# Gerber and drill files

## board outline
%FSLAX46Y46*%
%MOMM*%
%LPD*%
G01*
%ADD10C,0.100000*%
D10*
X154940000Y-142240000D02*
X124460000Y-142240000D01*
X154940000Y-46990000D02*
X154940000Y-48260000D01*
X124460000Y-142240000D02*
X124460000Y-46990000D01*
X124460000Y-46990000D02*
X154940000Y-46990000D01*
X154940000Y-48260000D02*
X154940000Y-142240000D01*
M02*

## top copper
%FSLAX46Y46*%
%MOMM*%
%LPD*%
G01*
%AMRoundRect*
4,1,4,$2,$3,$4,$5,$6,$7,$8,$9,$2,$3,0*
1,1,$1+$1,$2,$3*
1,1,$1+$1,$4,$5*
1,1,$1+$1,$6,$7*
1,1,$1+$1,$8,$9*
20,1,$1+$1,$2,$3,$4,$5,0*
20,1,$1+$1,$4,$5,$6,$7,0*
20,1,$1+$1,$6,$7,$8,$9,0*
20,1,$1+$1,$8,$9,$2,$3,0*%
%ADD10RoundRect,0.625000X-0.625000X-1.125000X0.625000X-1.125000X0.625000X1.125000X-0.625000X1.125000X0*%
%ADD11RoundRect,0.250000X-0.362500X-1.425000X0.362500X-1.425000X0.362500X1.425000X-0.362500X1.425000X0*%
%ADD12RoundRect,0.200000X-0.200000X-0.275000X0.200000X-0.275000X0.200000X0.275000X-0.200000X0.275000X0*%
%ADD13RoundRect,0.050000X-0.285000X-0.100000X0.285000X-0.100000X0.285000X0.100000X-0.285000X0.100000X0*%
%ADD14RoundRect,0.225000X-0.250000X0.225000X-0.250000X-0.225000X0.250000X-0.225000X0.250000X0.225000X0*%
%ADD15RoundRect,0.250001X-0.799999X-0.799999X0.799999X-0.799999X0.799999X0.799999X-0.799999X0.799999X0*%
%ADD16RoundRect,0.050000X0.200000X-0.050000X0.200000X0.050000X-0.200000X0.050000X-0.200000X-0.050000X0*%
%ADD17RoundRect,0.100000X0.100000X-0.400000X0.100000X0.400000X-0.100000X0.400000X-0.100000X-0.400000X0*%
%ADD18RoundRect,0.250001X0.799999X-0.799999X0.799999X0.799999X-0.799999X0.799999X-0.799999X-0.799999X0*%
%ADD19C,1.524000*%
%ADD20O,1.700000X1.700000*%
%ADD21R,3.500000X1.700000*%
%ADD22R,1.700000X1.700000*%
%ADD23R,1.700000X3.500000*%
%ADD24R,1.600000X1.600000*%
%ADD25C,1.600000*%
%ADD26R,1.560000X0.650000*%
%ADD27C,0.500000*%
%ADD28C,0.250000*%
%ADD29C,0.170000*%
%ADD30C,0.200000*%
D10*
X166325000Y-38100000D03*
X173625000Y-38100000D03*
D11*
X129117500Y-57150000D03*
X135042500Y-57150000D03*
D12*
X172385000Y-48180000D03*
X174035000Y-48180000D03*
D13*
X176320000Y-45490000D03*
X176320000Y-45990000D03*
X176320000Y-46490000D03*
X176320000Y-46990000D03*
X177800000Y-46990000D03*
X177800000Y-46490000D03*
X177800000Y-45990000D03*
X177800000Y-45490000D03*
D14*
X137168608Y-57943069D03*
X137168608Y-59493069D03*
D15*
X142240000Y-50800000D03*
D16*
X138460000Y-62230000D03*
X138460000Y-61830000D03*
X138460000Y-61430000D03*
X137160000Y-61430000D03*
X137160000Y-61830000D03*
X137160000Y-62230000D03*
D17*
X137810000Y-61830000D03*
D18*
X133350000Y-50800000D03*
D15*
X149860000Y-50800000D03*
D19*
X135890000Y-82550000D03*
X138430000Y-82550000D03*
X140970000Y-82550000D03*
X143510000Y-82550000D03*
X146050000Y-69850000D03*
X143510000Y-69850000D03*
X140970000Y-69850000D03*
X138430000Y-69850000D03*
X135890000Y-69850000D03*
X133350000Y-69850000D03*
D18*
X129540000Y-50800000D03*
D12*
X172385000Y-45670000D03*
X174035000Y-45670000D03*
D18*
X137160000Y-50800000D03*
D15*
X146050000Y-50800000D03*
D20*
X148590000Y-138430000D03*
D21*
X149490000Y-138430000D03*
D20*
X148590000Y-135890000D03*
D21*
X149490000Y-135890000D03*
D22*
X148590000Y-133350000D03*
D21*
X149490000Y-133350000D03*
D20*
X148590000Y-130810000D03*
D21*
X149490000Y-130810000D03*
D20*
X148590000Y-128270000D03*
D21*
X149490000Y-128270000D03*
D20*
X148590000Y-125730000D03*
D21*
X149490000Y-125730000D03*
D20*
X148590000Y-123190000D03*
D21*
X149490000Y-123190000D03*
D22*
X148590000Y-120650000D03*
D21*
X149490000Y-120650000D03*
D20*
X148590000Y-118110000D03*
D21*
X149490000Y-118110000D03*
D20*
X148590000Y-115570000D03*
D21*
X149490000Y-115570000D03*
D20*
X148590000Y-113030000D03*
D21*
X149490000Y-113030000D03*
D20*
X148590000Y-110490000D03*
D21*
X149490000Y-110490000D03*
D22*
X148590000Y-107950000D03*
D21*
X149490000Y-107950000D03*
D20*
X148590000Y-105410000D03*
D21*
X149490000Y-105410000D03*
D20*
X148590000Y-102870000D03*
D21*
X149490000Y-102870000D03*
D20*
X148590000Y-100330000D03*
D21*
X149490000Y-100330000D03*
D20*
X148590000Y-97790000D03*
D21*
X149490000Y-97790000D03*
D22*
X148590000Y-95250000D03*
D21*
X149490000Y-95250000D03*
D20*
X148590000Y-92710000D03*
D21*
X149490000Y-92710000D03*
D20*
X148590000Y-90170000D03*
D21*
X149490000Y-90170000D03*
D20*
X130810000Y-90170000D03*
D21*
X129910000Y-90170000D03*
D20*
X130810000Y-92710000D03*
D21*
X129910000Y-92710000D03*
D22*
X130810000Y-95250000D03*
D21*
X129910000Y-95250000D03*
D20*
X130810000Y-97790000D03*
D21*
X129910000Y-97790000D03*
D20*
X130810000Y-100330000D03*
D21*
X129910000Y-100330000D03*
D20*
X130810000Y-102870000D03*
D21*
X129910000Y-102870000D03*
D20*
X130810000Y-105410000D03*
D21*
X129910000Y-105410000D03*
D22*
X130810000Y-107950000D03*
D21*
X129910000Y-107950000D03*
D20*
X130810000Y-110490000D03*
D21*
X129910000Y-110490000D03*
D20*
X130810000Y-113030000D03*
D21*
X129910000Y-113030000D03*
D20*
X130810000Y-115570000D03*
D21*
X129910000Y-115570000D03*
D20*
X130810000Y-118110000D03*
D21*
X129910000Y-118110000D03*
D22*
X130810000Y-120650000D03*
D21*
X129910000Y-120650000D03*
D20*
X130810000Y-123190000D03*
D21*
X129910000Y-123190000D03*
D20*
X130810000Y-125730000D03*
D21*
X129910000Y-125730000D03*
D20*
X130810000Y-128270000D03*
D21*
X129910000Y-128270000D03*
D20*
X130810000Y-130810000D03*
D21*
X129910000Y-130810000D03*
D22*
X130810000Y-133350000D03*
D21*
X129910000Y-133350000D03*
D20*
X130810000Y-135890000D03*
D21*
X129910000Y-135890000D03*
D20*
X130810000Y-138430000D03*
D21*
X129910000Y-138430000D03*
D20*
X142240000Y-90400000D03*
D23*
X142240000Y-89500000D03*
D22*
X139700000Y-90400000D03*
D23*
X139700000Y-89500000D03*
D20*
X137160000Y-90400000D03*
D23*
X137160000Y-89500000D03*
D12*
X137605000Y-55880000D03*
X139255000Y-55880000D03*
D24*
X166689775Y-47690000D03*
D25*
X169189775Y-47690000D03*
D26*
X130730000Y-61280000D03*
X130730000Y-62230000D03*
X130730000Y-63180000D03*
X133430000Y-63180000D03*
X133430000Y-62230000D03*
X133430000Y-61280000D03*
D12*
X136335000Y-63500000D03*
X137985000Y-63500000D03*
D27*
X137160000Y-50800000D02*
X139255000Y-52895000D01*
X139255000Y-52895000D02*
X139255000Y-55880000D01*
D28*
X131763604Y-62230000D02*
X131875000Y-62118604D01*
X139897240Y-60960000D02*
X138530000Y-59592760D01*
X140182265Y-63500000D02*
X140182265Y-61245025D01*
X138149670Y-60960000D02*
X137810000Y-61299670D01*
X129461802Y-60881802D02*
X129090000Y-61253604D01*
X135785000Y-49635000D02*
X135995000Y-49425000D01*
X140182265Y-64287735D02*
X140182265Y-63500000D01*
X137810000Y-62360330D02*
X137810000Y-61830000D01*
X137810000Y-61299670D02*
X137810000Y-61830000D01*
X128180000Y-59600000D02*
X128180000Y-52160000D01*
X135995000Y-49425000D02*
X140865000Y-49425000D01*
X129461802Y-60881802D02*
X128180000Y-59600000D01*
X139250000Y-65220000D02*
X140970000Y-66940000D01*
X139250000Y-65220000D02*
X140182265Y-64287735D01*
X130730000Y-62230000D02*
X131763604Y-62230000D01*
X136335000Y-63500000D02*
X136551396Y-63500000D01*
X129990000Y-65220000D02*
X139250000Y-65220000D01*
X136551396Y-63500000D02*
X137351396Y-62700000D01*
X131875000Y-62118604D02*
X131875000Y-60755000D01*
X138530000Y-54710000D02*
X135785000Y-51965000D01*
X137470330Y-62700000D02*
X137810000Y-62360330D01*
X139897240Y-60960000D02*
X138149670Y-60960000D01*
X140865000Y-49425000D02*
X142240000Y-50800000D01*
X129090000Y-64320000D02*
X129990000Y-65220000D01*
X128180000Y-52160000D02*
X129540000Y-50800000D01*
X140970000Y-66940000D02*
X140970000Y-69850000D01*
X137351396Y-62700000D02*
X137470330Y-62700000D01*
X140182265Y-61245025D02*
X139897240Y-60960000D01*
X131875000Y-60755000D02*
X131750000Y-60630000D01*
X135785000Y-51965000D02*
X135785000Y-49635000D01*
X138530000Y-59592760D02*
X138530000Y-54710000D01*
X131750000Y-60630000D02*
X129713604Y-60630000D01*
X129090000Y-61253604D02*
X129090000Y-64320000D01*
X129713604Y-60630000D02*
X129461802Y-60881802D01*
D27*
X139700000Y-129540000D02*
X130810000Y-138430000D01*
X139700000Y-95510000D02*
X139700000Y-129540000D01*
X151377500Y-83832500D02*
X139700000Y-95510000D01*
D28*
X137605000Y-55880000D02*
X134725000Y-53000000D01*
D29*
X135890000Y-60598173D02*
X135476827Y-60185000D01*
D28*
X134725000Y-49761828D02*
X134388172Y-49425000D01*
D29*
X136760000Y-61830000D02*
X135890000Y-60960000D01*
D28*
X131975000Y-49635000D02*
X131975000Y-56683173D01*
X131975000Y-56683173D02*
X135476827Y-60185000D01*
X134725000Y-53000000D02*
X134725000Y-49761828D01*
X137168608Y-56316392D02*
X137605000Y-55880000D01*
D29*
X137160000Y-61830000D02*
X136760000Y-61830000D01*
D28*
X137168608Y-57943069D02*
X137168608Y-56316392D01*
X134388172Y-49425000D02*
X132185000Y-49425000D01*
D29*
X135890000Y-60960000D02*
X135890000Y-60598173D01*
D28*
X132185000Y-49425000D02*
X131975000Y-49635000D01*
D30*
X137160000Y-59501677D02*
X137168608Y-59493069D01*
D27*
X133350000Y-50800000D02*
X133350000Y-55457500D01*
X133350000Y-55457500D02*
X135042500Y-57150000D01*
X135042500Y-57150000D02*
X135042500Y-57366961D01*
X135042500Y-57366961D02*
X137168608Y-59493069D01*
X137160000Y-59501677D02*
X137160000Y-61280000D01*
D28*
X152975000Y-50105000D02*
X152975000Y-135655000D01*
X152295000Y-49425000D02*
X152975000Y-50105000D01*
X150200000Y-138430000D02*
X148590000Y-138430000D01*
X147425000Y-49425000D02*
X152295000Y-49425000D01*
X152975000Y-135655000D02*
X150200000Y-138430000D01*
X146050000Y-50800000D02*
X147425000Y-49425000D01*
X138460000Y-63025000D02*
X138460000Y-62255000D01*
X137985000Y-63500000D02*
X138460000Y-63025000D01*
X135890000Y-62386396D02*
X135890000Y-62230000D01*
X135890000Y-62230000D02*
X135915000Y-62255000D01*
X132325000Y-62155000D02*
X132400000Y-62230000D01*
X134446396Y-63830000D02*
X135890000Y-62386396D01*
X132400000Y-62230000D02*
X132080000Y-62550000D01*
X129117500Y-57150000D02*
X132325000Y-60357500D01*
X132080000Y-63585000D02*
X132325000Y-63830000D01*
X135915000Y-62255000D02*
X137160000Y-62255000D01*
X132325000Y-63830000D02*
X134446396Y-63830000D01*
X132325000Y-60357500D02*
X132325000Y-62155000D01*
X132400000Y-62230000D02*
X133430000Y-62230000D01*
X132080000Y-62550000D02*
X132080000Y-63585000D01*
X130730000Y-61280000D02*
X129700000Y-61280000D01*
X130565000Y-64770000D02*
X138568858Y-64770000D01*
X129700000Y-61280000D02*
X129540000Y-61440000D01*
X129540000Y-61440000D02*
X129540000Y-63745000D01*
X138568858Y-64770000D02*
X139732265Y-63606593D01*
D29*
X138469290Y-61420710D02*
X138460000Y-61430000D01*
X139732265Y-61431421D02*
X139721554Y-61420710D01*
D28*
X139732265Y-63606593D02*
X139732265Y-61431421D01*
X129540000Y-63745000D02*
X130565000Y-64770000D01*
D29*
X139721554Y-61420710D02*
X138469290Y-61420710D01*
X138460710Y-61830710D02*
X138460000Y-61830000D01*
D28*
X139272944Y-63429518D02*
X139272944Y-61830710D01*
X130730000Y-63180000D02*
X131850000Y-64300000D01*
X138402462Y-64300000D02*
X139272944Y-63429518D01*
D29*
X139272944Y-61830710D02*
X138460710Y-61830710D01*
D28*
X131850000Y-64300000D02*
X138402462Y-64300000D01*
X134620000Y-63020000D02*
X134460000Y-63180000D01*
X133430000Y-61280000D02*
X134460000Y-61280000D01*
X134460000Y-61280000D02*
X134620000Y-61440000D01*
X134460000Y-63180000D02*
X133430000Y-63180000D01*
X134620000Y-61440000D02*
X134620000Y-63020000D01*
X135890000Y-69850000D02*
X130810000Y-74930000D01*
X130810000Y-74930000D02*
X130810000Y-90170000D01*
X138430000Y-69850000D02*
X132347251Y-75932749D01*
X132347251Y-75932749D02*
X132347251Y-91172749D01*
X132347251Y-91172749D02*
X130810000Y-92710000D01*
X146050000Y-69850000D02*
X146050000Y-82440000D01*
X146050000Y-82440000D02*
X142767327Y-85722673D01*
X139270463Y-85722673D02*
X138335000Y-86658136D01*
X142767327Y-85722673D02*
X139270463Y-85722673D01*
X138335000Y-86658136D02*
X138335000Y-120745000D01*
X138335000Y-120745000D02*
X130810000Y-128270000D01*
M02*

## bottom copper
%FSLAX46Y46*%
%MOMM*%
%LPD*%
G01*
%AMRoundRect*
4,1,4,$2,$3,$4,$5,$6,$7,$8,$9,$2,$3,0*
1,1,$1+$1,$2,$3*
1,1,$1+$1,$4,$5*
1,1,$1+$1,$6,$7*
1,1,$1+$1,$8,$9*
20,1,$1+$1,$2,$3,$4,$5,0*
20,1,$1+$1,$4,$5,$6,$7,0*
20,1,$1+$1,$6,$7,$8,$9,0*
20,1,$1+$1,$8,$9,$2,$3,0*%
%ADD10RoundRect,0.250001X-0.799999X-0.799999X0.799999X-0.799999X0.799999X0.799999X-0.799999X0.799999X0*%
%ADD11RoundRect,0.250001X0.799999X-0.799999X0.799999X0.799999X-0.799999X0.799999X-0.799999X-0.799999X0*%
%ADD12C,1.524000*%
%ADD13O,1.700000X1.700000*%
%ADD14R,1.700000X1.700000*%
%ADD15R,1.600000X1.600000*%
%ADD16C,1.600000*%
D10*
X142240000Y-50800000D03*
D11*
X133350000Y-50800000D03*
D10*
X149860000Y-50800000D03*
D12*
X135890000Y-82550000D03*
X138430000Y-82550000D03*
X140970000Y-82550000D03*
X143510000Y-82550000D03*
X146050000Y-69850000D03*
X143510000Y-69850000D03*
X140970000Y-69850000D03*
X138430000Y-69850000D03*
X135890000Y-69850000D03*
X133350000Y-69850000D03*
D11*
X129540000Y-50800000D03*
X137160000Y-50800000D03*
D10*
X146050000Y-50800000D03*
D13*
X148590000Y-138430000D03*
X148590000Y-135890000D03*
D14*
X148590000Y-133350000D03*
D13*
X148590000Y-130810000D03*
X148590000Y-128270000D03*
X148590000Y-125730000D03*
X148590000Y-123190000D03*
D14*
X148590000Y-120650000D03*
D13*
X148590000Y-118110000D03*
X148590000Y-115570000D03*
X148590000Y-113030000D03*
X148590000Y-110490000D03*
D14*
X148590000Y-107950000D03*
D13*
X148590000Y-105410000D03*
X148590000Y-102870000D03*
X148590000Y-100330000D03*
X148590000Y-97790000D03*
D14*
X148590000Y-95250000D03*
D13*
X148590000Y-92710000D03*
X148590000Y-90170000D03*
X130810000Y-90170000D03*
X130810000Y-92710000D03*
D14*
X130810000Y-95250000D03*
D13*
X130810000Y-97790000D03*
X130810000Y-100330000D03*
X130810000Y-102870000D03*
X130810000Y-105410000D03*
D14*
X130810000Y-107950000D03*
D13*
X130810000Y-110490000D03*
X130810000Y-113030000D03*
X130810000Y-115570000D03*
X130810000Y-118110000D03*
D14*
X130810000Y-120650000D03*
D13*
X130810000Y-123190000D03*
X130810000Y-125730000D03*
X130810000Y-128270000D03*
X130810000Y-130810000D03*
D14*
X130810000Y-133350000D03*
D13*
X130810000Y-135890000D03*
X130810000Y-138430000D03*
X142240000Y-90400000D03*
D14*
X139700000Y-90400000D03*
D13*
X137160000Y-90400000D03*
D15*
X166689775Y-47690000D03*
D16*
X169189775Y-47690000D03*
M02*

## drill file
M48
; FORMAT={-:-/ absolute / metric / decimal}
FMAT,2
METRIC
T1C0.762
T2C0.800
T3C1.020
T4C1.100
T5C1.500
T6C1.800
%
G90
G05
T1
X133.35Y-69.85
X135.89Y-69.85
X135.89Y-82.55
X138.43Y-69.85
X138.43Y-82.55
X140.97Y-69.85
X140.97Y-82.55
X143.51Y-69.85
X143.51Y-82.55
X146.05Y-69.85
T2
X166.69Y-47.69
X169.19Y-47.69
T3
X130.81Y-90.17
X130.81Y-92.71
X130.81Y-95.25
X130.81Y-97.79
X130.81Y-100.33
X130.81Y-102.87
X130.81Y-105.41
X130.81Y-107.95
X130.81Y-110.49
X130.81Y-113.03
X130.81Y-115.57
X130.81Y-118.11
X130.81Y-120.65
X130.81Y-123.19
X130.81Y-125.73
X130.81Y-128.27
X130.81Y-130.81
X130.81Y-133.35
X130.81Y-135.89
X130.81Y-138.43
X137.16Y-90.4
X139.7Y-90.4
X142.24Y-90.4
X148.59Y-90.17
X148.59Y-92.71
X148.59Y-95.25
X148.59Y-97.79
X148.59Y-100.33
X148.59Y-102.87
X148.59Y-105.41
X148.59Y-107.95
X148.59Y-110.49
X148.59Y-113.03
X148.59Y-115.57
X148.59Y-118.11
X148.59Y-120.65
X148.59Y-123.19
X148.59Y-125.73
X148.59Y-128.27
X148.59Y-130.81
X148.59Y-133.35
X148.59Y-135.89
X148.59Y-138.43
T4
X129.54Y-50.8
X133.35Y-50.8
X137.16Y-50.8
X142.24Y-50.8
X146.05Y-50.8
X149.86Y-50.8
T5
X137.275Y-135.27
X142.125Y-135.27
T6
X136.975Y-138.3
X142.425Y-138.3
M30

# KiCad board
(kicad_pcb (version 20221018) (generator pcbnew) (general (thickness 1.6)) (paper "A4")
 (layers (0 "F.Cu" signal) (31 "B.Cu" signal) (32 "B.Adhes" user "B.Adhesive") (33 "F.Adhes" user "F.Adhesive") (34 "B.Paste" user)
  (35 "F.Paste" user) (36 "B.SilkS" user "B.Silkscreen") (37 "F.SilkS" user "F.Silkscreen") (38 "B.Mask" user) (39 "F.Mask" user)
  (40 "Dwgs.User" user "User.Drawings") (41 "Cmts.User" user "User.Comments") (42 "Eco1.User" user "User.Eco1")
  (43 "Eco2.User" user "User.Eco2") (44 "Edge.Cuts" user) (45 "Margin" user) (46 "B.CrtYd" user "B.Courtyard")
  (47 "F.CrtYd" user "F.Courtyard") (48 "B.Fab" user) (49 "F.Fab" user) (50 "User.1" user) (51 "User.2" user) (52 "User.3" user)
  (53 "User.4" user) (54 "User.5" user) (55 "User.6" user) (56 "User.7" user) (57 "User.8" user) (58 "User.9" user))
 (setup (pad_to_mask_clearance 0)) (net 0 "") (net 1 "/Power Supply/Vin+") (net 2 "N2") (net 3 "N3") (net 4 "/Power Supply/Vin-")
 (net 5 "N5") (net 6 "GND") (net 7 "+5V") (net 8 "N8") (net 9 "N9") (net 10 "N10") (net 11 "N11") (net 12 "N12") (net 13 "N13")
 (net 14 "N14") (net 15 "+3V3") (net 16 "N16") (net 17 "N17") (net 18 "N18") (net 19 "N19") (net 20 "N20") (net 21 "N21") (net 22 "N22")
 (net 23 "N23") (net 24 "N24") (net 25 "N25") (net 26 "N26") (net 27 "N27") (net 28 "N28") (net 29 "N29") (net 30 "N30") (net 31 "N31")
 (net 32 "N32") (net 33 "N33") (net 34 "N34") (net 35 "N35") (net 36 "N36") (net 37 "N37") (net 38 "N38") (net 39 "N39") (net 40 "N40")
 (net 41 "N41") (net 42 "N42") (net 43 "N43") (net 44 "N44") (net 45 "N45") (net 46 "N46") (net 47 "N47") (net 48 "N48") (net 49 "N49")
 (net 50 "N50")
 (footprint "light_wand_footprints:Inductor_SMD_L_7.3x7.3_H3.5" (layer "F.Cu") (at 169.975 38.1)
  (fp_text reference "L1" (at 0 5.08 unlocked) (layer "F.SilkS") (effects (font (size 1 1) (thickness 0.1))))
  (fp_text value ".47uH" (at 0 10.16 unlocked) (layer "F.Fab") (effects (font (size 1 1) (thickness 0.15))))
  (pad "1" smd roundrect (at -3.65 0) (size 2.5 3.5) (layers "F.Cu" "F.Paste" "F.Mask") (roundrect_rratio 0.25) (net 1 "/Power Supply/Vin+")
   (thermal_bridge_angle 45))
  (pad "2" smd roundrect (at 3.65 0) (size 2.5 3.5) (layers "F.Cu" "F.Paste" "F.Mask") (roundrect_rratio 0.25) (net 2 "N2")
   (thermal_bridge_angle 45)))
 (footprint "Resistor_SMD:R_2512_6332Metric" (layer "F.Cu") (at 132.08 57.15)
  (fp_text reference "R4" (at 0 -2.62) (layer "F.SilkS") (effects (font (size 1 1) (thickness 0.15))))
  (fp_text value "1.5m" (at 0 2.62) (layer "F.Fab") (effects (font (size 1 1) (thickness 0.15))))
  (pad "1" smd roundrect (at -2.9625 0) (size 1.225 3.35) (layers "F.Cu" "F.Paste" "F.Mask") (roundrect_rratio 0.204082) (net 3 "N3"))
  (pad "2" smd roundrect (at 2.9625 0) (size 1.225 3.35) (layers "F.Cu" "F.Paste" "F.Mask") (roundrect_rratio 0.204082)
   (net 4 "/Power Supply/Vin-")))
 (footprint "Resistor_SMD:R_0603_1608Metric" (layer "F.Cu") (at 173.21 48.18)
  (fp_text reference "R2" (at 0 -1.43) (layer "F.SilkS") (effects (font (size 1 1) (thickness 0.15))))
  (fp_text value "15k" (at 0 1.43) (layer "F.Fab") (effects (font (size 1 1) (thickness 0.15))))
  (pad "1" smd roundrect (at -0.825 0) (size 0.8 0.95) (layers "F.Cu" "F.Paste" "F.Mask") (roundrect_rratio 0.25) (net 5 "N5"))
  (pad "2" smd roundrect (at 0.825 0) (size 0.8 0.95) (layers "F.Cu" "F.Paste" "F.Mask") (roundrect_rratio 0.25) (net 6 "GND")))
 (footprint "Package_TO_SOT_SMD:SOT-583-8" (layer "F.Cu") (at 177.06 46.24)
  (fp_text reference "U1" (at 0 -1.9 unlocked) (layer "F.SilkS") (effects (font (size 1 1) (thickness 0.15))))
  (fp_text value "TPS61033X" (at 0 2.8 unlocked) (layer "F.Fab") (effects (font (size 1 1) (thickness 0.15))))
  (pad "1" smd roundrect (at -0.74 -0.75) (size 0.67 0.3) (layers "F.Cu" "F.Paste" "F.Mask") (roundrect_rratio 0.1666666667)
   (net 1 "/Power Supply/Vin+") (thermal_bridge_angle 45))
  (pad "2" smd roundrect (at -0.74 -0.25) (size 0.67 0.3) (layers "F.Cu" "F.Paste" "F.Mask") (roundrect_rratio 0.1666666667)
   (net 1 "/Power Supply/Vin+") (thermal_bridge_angle 45))
  (pad "3" smd roundrect (at -0.74 0.25) (size 0.67 0.3) (layers "F.Cu" "F.Paste" "F.Mask") (roundrect_rratio 0.1666666667)
   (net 1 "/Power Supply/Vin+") (thermal_bridge_angle 45))
  (pad "4" smd roundrect (at -0.74 0.75) (size 0.67 0.3) (layers "F.Cu" "F.Paste" "F.Mask") (roundrect_rratio 0.1666666667) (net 6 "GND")
   (thermal_bridge_angle 45))
  (pad "5" smd roundrect (at 0.74 0.75) (size 0.67 0.3) (layers "F.Cu" "F.Paste" "F.Mask") (roundrect_rratio 0.1666666667) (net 5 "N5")
   (thermal_bridge_angle 45))
  (pad "6" smd roundrect (at 0.74 0.25) (size 0.67 0.3) (layers "F.Cu" "F.Paste" "F.Mask") (roundrect_rratio 0.1666666667) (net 6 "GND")
   (thermal_bridge_angle 45))
  (pad "7" smd roundrect (at 0.74 -0.25) (size 0.67 0.3) (layers "F.Cu" "F.Paste" "F.Mask") (roundrect_rratio 0.1666666667) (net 2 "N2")
   (thermal_bridge_angle 45))
  (pad "8" smd roundrect (at 0.74 -0.75) (size 0.67 0.3) (layers "F.Cu" "F.Paste" "F.Mask") (roundrect_rratio 0.1666666667) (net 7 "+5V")
   (thermal_bridge_angle 45)))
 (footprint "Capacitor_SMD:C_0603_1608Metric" (layer "F.Cu") (at 137.168608 58.718069 -90)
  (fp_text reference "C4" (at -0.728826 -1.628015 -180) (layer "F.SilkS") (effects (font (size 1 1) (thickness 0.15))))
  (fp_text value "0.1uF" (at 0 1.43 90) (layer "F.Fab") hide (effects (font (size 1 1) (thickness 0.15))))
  (pad "1" smd roundrect (at -0.775 0 270) (size 0.9 0.95) (layers "F.Cu" "F.Paste" "F.Mask") (roundrect_rratio 0.25) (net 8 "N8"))
  (pad "2" smd roundrect (at 0.775 0 270) (size 0.9 0.95) (layers "F.Cu" "F.Paste" "F.Mask") (roundrect_rratio 0.25)
   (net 4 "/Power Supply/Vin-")))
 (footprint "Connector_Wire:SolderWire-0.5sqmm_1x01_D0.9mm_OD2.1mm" (layer "F.Cu") (at 142.24 50.8)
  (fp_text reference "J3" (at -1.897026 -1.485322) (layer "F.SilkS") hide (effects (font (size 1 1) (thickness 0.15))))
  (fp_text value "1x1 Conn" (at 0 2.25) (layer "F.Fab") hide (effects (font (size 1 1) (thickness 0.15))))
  (pad "1" thru_hole roundrect (at 0 0) (size 2.1 2.1) (drill 1.1) (layers "*.Cu" "*.Mask") (roundrect_rratio 0.119048) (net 6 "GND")))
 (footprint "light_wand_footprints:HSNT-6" (layer "F.Cu") (at 137.81 61.83 180)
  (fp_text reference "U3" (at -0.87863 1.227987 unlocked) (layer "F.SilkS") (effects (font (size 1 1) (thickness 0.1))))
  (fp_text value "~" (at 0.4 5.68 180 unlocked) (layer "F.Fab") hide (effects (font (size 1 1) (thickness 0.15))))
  (pad "1" smd roundrect (at -0.65 -0.4 90) (size 0.2 0.5) (layers "F.Cu" "F.Paste" "F.Mask") (roundrect_rratio 0.25) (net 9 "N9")
   (thermal_bridge_angle 45))
  (pad "2" smd roundrect (at -0.65 0 90) (size 0.2 0.5) (layers "F.Cu" "F.Paste" "F.Mask") (roundrect_rratio 0.25) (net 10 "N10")
   (thermal_bridge_angle 45))
  (pad "3" smd roundrect (at -0.65 0.4 90) (size 0.2 0.5) (layers "F.Cu" "F.Paste" "F.Mask") (roundrect_rratio 0.25) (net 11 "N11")
   (thermal_bridge_angle 45))
  (pad "4" smd roundrect (at 0.65 0.4 90) (size 0.2 0.5) (layers "F.Cu" "F.Paste" "F.Mask") (roundrect_rratio 0.25)
   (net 4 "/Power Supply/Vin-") (thermal_bridge_angle 45))
  (pad "5" smd roundrect (at 0.65 0 90) (size 0.2 0.5) (layers "F.Cu" "F.Paste" "F.Mask") (roundrect_rratio 0.25) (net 8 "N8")
   (thermal_bridge_angle 45))
  (pad "6" smd roundrect (at 0.65 -0.4 90) (size 0.2 0.5) (layers "F.Cu" "F.Paste" "F.Mask") (roundrect_rratio 0.25) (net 3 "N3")
   (thermal_bridge_angle 45))
  (pad "7" smd roundrect (at 0 0 90) (size 1 0.4) (layers "F.Cu" "F.Paste" "F.Mask") (roundrect_rratio 0.25) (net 6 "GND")
   (thermal_bridge_angle 45)))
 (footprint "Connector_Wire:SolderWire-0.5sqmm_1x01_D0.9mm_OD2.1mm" (layer "F.Cu") (at 133.35 50.8 90)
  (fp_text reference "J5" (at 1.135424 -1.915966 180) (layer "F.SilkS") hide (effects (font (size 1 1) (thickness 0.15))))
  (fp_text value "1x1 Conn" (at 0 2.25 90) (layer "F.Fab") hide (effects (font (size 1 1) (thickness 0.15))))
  (pad "1" thru_hole roundrect (at 0 0 90) (size 2.1 2.1) (drill 1.1) (layers "*.Cu" "*.Mask") (roundrect_rratio 0.119048)
   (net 4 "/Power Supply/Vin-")))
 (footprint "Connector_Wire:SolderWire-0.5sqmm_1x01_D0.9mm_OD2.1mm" (layer "F.Cu") (at 149.86 50.8)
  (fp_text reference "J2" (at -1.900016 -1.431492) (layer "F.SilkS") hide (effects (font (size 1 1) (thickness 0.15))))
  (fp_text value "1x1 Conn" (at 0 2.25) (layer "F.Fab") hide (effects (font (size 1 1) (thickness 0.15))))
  (pad "1" thru_hole roundrect (at 0 0) (size 2.1 2.1) (drill 1.1) (layers "*.Cu" "*.Mask") (roundrect_rratio 0.119048) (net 7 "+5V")))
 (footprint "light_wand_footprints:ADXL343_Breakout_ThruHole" (layer "F.Cu") (at 151.13 74.93 90)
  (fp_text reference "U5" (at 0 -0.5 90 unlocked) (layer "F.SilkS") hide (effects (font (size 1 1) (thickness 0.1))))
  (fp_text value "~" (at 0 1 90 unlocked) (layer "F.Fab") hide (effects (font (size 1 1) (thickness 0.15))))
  (pad "1" thru_hole circle (at -7.62 -15.24 90) (size 1.524 1.524) (drill 0.762) (layers "*.Cu" "*.Mask") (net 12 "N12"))
  (pad "2" thru_hole circle (at -7.62 -12.7 90) (size 1.524 1.524) (drill 0.762) (layers "*.Cu" "*.Mask") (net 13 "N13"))
  (pad "3" thru_hole circle (at -7.62 -10.16 90) (size 1.524 1.524) (drill 0.762) (layers "*.Cu" "*.Mask") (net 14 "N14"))
  (pad "4" thru_hole circle (at -7.62 -7.62 90) (size 1.524 1.524) (drill 0.762) (layers "*.Cu" "*.Mask") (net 6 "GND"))
  (pad "5" thru_hole circle (at 5.08 -5.08 90) (size 1.524 1.524) (drill 0.762) (layers "*.Cu" "*.Mask") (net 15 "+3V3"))
  (pad "6" thru_hole circle (at 5.08 -7.62 90) (size 1.524 1.524) (drill 0.762) (layers "*.Cu" "*.Mask") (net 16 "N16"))
  (pad "7" thru_hole circle (at 5.08 -10.16 90) (size 1.524 1.524) (drill 0.762) (layers "*.Cu" "*.Mask") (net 6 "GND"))
  (pad "8" thru_hole circle (at 5.08 -12.7 90) (size 1.524 1.524) (drill 0.762) (layers "*.Cu" "*.Mask") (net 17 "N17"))
  (pad "9" thru_hole circle (at 5.08 -15.24 90) (size 1.524 1.524) (drill 0.762) (layers "*.Cu" "*.Mask") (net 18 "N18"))
  (pad "10" thru_hole circle (at 5.08 -17.78 90) (size 1.524 1.524) (drill 0.762) (layers "*.Cu" "*.Mask") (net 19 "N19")))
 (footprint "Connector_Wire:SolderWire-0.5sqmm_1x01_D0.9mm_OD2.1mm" (layer "F.Cu") (at 129.54 50.8 90)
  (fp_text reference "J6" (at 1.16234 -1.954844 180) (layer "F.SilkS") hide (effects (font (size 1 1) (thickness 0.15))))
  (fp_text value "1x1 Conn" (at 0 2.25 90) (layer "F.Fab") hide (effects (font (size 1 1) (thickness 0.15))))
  (pad "1" thru_hole roundrect (at 0 0 90) (size 2.1 2.1) (drill 1.1) (layers "*.Cu" "*.Mask") (roundrect_rratio 0.119048) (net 6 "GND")))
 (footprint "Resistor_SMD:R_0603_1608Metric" (layer "F.Cu") (at 173.21 45.67)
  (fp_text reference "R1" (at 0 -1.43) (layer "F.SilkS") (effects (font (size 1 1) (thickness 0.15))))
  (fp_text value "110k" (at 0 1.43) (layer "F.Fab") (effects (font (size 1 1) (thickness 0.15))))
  (pad "1" smd roundrect (at -0.825 0) (size 0.8 0.95) (layers "F.Cu" "F.Paste" "F.Mask") (roundrect_rratio 0.25) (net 7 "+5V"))
  (pad "2" smd roundrect (at 0.825 0) (size 0.8 0.95) (layers "F.Cu" "F.Paste" "F.Mask") (roundrect_rratio 0.25) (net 5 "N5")))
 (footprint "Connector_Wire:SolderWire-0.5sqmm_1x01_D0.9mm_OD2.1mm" (layer "F.Cu") (at 137.16 50.8 90)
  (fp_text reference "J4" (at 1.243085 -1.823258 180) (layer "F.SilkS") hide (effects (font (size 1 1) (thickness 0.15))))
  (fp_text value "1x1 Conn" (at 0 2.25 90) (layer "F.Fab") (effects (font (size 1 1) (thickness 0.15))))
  (pad "1" thru_hole roundrect (at 0 0 90) (size 2.1 2.1) (drill 1.1) (layers "*.Cu" "*.Mask") (roundrect_rratio 0.119048)
   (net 1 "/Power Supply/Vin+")))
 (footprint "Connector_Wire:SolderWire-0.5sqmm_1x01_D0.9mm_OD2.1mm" (layer "F.Cu") (at 146.05 50.8)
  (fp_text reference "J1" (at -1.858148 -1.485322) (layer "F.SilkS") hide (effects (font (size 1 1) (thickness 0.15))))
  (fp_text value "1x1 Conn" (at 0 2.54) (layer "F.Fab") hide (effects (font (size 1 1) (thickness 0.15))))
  (pad "1" thru_hole roundrect (at 0 0) (size 2.1 2.1) (drill 1.1) (layers "*.Cu" "*.Mask") (roundrect_rratio 0.119048) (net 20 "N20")))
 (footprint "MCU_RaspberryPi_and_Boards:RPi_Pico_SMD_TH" (layer "F.Cu") (at 139.7 114.3 180)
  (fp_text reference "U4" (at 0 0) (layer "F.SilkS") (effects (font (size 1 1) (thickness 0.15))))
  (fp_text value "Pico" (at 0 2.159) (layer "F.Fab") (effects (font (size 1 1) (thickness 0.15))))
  (pad "" np_thru_hole oval (at -2.725 -24 180) (size 1.8 1.8) (drill 1.8) (layers "*.Cu" "*.Mask"))
  (pad "" np_thru_hole oval (at -2.425 -20.97 180) (size 1.5 1.5) (drill 1.5) (layers "*.Cu" "*.Mask"))
  (pad "" np_thru_hole oval (at 2.425 -20.97 180) (size 1.5 1.5) (drill 1.5) (layers "*.Cu" "*.Mask"))
  (pad "" np_thru_hole oval (at 2.725 -24 180) (size 1.8 1.8) (drill 1.8) (layers "*.Cu" "*.Mask"))
  (pad "1" thru_hole oval (at -8.89 -24.13 180) (size 1.7 1.7) (drill 1.02) (layers "*.Cu" "*.Mask") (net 20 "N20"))
  (pad "1" smd rect (at -8.89 -24.13 180) (size 3.5 1.7) (drill (offset -0.9 0)) (layers "F.Cu" "F.Mask") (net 20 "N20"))
  (pad "2" thru_hole oval (at -8.89 -21.59 180) (size 1.7 1.7) (drill 1.02) (layers "*.Cu" "*.Mask") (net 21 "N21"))
  (pad "2" smd rect (at -8.89 -21.59 180) (size 3.5 1.7) (drill (offset -0.9 0)) (layers "F.Cu" "F.Mask") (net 21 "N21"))
  (pad "3" thru_hole rect (at -8.89 -19.05 180) (size 1.7 1.7) (drill 1.02) (layers "*.Cu" "*.Mask") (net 6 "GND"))
  (pad "3" smd rect (at -8.89 -19.05 180) (size 3.5 1.7) (drill (offset -0.9 0)) (layers "F.Cu" "F.Mask") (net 6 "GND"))
  (pad "4" thru_hole oval (at -8.89 -16.51 180) (size 1.7 1.7) (drill 1.02) (layers "*.Cu" "*.Mask") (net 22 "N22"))
  (pad "4" smd rect (at -8.89 -16.51 180) (size 3.5 1.7) (drill (offset -0.9 0)) (layers "F.Cu" "F.Mask") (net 22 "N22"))
  (pad "5" thru_hole oval (at -8.89 -13.97 180) (size 1.7 1.7) (drill 1.02) (layers "*.Cu" "*.Mask") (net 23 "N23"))
  (pad "5" smd rect (at -8.89 -13.97 180) (size 3.5 1.7) (drill (offset -0.9 0)) (layers "F.Cu" "F.Mask") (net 23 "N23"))
  (pad "6" thru_hole oval (at -8.89 -11.43 180) (size 1.7 1.7) (drill 1.02) (layers "*.Cu" "*.Mask") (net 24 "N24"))
  (pad "6" smd rect (at -8.89 -11.43 180) (size 3.5 1.7) (drill (offset -0.9 0)) (layers "F.Cu" "F.Mask") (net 24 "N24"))
  (pad "7" thru_hole oval (at -8.89 -8.89 180) (size 1.7 1.7) (drill 1.02) (layers "*.Cu" "*.Mask") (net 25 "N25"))
  (pad "7" smd rect (at -8.89 -8.89 180) (size 3.5 1.7) (drill (offset -0.9 0)) (layers "F.Cu" "F.Mask") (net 25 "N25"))
  (pad "8" thru_hole rect (at -8.89 -6.35 180) (size 1.7 1.7) (drill 1.02) (layers "*.Cu" "*.Mask") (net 6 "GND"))
  (pad "8" smd rect (at -8.89 -6.35 180) (size 3.5 1.7) (drill (offset -0.9 0)) (layers "F.Cu" "F.Mask") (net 6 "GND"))
  (pad "9" thru_hole oval (at -8.89 -3.81 180) (size 1.7 1.7) (drill 1.02) (layers "*.Cu" "*.Mask") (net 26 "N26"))
  (pad "9" smd rect (at -8.89 -3.81 180) (size 3.5 1.7) (drill (offset -0.9 0)) (layers "F.Cu" "F.Mask") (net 26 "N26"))
  (pad "10" thru_hole oval (at -8.89 -1.27 180) (size 1.7 1.7) (drill 1.02) (layers "*.Cu" "*.Mask") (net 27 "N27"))
  (pad "10" smd rect (at -8.89 -1.27 180) (size 3.5 1.7) (drill (offset -0.9 0)) (layers "F.Cu" "F.Mask") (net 27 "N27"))
  (pad "11" thru_hole oval (at -8.89 1.27 180) (size 1.7 1.7) (drill 1.02) (layers "*.Cu" "*.Mask") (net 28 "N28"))
  (pad "11" smd rect (at -8.89 1.27 180) (size 3.5 1.7) (drill (offset -0.9 0)) (layers "F.Cu" "F.Mask") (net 28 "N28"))
  (pad "12" thru_hole oval (at -8.89 3.81 180) (size 1.7 1.7) (drill 1.02) (layers "*.Cu" "*.Mask") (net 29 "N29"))
  (pad "12" smd rect (at -8.89 3.81 180) (size 3.5 1.7) (drill (offset -0.9 0)) (layers "F.Cu" "F.Mask") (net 29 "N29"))
  (pad "13" thru_hole rect (at -8.89 6.35 180) (size 1.7 1.7) (drill 1.02) (layers "*.Cu" "*.Mask") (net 6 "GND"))
  (pad "13" smd rect (at -8.89 6.35 180) (size 3.5 1.7) (drill (offset -0.9 0)) (layers "F.Cu" "F.Mask") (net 6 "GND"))
  (pad "14" thru_hole oval (at -8.89 8.89 180) (size 1.7 1.7) (drill 1.02) (layers "*.Cu" "*.Mask") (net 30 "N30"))
  (pad "14" smd rect (at -8.89 8.89 180) (size 3.5 1.7) (drill (offset -0.9 0)) (layers "F.Cu" "F.Mask") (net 30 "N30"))
  (pad "15" thru_hole oval (at -8.89 11.43 180) (size 1.7 1.7) (drill 1.02) (layers "*.Cu" "*.Mask") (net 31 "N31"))
  (pad "15" smd rect (at -8.89 11.43 180) (size 3.5 1.7) (drill (offset -0.9 0)) (layers "F.Cu" "F.Mask") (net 31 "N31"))
  (pad "16" thru_hole oval (at -8.89 13.97 180) (size 1.7 1.7) (drill 1.02) (layers "*.Cu" "*.Mask") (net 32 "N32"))
  (pad "16" smd rect (at -8.89 13.97 180) (size 3.5 1.7) (drill (offset -0.9 0)) (layers "F.Cu" "F.Mask") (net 32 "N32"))
  (pad "17" thru_hole oval (at -8.89 16.51 180) (size 1.7 1.7) (drill 1.02) (layers "*.Cu" "*.Mask") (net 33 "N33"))
  (pad "17" smd rect (at -8.89 16.51 180) (size 3.5 1.7) (drill (offset -0.9 0)) (layers "F.Cu" "F.Mask") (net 33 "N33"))
  (pad "18" thru_hole rect (at -8.89 19.05 180) (size 1.7 1.7) (drill 1.02) (layers "*.Cu" "*.Mask") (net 6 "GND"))
  (pad "18" smd rect (at -8.89 19.05 180) (size 3.5 1.7) (drill (offset -0.9 0)) (layers "F.Cu" "F.Mask") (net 6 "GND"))
  (pad "19" thru_hole oval (at -8.89 21.59 180) (size 1.7 1.7) (drill 1.02) (layers "*.Cu" "*.Mask") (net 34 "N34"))
  (pad "19" smd rect (at -8.89 21.59 180) (size 3.5 1.7) (drill (offset -0.9 0)) (layers "F.Cu" "F.Mask") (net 34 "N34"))
  (pad "20" thru_hole oval (at -8.89 24.13 180) (size 1.7 1.7) (drill 1.02) (layers "*.Cu" "*.Mask") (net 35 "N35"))
  (pad "20" smd rect (at -8.89 24.13 180) (size 3.5 1.7) (drill (offset -0.9 0)) (layers "F.Cu" "F.Mask") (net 35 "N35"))
  (pad "21" thru_hole oval (at 8.89 24.13 180) (size 1.7 1.7) (drill 1.02) (layers "*.Cu" "*.Mask") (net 18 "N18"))
  (pad "21" smd rect (at 8.89 24.13 180) (size 3.5 1.7) (drill (offset 0.9 0)) (layers "F.Cu" "F.Mask") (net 18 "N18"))
  (pad "22" thru_hole oval (at 8.89 21.59 180) (size 1.7 1.7) (drill 1.02) (layers "*.Cu" "*.Mask") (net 17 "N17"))
  (pad "22" smd rect (at 8.89 21.59 180) (size 3.5 1.7) (drill (offset 0.9 0)) (layers "F.Cu" "F.Mask") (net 17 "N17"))
  (pad "23" thru_hole rect (at 8.89 19.05 180) (size 1.7 1.7) (drill 1.02) (layers "*.Cu" "*.Mask") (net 6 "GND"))
  (pad "23" smd rect (at 8.89 19.05 180) (size 3.5 1.7) (drill (offset 0.9 0)) (layers "F.Cu" "F.Mask") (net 6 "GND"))
  (pad "24" thru_hole oval (at 8.89 16.51 180) (size 1.7 1.7) (drill 1.02) (layers "*.Cu" "*.Mask") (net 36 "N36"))
  (pad "24" smd rect (at 8.89 16.51 180) (size 3.5 1.7) (drill (offset 0.9 0)) (layers "F.Cu" "F.Mask") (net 36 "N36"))
  (pad "25" thru_hole oval (at 8.89 13.97 180) (size 1.7 1.7) (drill 1.02) (layers "*.Cu" "*.Mask") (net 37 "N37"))
  (pad "25" smd rect (at 8.89 13.97 180) (size 3.5 1.7) (drill (offset 0.9 0)) (layers "F.Cu" "F.Mask") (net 37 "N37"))
  (pad "26" thru_hole oval (at 8.89 11.43 180) (size 1.7 1.7) (drill 1.02) (layers "*.Cu" "*.Mask") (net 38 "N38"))
  (pad "26" smd rect (at 8.89 11.43 180) (size 3.5 1.7) (drill (offset 0.9 0)) (layers "F.Cu" "F.Mask") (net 38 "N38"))
  (pad "27" thru_hole oval (at 8.89 8.89 180) (size 1.7 1.7) (drill 1.02) (layers "*.Cu" "*.Mask") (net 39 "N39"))
  (pad "27" smd rect (at 8.89 8.89 180) (size 3.5 1.7) (drill (offset 0.9 0)) (layers "F.Cu" "F.Mask") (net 39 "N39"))
  (pad "28" thru_hole rect (at 8.89 6.35 180) (size 1.7 1.7) (drill 1.02) (layers "*.Cu" "*.Mask") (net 6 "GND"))
  (pad "28" smd rect (at 8.89 6.35 180) (size 3.5 1.7) (drill (offset 0.9 0)) (layers "F.Cu" "F.Mask") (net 6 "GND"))
  (pad "29" thru_hole oval (at 8.89 3.81 180) (size 1.7 1.7) (drill 1.02) (layers "*.Cu" "*.Mask") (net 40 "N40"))
  (pad "29" smd rect (at 8.89 3.81 180) (size 3.5 1.7) (drill (offset 0.9 0)) (layers "F.Cu" "F.Mask") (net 40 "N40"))
  (pad "30" thru_hole oval (at 8.89 1.27 180) (size 1.7 1.7) (drill 1.02) (layers "*.Cu" "*.Mask") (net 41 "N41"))
  (pad "30" smd rect (at 8.89 1.27 180) (size 3.5 1.7) (drill (offset 0.9 0)) (layers "F.Cu" "F.Mask") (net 41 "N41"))
  (pad "31" thru_hole oval (at 8.89 -1.27 180) (size 1.7 1.7) (drill 1.02) (layers "*.Cu" "*.Mask") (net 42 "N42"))
  (pad "31" smd rect (at 8.89 -1.27 180) (size 3.5 1.7) (drill (offset 0.9 0)) (layers "F.Cu" "F.Mask") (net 42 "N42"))
  (pad "32" thru_hole oval (at 8.89 -3.81 180) (size 1.7 1.7) (drill 1.02) (layers "*.Cu" "*.Mask") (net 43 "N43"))
  (pad "32" smd rect (at 8.89 -3.81 180) (size 3.5 1.7) (drill (offset 0.9 0)) (layers "F.Cu" "F.Mask") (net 43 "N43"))
  (pad "33" thru_hole rect (at 8.89 -6.35 180) (size 1.7 1.7) (drill 1.02) (layers "*.Cu" "*.Mask") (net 6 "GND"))
  (pad "33" smd rect (at 8.89 -6.35 180) (size 3.5 1.7) (drill (offset 0.9 0)) (layers "F.Cu" "F.Mask") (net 6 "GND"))
  (pad "34" thru_hole oval (at 8.89 -8.89 180) (size 1.7 1.7) (drill 1.02) (layers "*.Cu" "*.Mask") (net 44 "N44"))
  (pad "34" smd rect (at 8.89 -8.89 180) (size 3.5 1.7) (drill (offset 0.9 0)) (layers "F.Cu" "F.Mask") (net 44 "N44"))
  (pad "35" thru_hole oval (at 8.89 -11.43 180) (size 1.7 1.7) (drill 1.02) (layers "*.Cu" "*.Mask") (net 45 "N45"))
  (pad "35" smd rect (at 8.89 -11.43 180) (size 3.5 1.7) (drill (offset 0.9 0)) (layers "F.Cu" "F.Mask") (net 45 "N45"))
  (pad "36" thru_hole oval (at 8.89 -13.97 180) (size 1.7 1.7) (drill 1.02) (layers "*.Cu" "*.Mask") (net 15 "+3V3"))
  (pad "36" smd rect (at 8.89 -13.97 180) (size 3.5 1.7) (drill (offset 0.9 0)) (layers "F.Cu" "F.Mask") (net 15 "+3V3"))
  (pad "37" thru_hole oval (at 8.89 -16.51 180) (size 1.7 1.7) (drill 1.02) (layers "*.Cu" "*.Mask") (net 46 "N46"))
  (pad "37" smd rect (at 8.89 -16.51 180) (size 3.5 1.7) (drill (offset 0.9 0)) (layers "F.Cu" "F.Mask") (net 46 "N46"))
  (pad "38" thru_hole rect (at 8.89 -19.05 180) (size 1.7 1.7) (drill 1.02) (layers "*.Cu" "*.Mask") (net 6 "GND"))
  (pad "38" smd rect (at 8.89 -19.05 180) (size 3.5 1.7) (drill (offset 0.9 0)) (layers "F.Cu" "F.Mask") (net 6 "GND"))
  (pad "39" thru_hole oval (at 8.89 -21.59 180) (size 1.7 1.7) (drill 1.02) (layers "*.Cu" "*.Mask") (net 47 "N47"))
  (pad "39" smd rect (at 8.89 -21.59 180) (size 3.5 1.7) (drill (offset 0.9 0)) (layers "F.Cu" "F.Mask") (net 47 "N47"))
  (pad "40" thru_hole oval (at 8.89 -24.13 180) (size 1.7 1.7) (drill 1.02) (layers "*.Cu" "*.Mask") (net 7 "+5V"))
  (pad "40" smd rect (at 8.89 -24.13 180) (size 3.5 1.7) (drill (offset 0.9 0)) (layers "F.Cu" "F.Mask") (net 7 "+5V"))
  (pad "41" thru_hole oval (at -2.54 23.9 180) (size 1.7 1.7) (drill 1.02) (layers "*.Cu" "*.Mask") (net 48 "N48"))
  (pad "41" smd rect (at -2.54 23.9 270) (size 3.5 1.7) (drill (offset -0.9 0)) (layers "F.Cu" "F.Mask") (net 48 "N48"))
  (pad "42" thru_hole rect (at 0 23.9 180) (size 1.7 1.7) (drill 1.02) (layers "*.Cu" "*.Mask") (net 6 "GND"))
  (pad "42" smd rect (at 0 23.9 270) (size 3.5 1.7) (drill (offset -0.9 0)) (layers "F.Cu" "F.Mask") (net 6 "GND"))
  (pad "43" thru_hole oval (at 2.54 23.9 180) (size 1.7 1.7) (drill 1.02) (layers "*.Cu" "*.Mask") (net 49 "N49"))
  (pad "43" smd rect (at 2.54 23.9 270) (size 3.5 1.7) (drill (offset -0.9 0)) (layers "F.Cu" "F.Mask") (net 49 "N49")))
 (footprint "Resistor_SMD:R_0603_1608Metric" (layer "F.Cu") (at 138.43 55.88)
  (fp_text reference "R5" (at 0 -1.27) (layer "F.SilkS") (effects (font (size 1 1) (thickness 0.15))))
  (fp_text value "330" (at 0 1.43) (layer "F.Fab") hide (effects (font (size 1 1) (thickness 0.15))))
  (pad "1" smd roundrect (at -0.825 0) (size 0.8 0.95) (layers "F.Cu" "F.Paste" "F.Mask") (roundrect_rratio 0.25) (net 8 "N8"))
  (pad "2" smd roundrect (at 0.825 0) (size 0.8 0.95) (layers "F.Cu" "F.Paste" "F.Mask") (roundrect_rratio 0.25)
   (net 1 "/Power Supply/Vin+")))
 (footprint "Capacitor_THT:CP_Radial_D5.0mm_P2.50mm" (layer "F.Cu") (at 166.689775 47.69)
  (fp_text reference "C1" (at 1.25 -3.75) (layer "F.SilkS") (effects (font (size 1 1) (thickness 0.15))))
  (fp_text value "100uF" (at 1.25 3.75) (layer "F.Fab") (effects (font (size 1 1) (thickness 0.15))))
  (pad "1" thru_hole rect (at 0 0) (size 1.6 1.6) (drill 0.8) (layers "*.Cu" "*.Mask") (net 1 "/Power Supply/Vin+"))
  (pad "2" thru_hole circle (at 2.5 0) (size 1.6 1.6) (drill 0.8) (layers "*.Cu" "*.Mask") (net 6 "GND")))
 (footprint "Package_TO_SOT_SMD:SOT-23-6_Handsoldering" (layer "F.Cu") (at 132.08 62.23)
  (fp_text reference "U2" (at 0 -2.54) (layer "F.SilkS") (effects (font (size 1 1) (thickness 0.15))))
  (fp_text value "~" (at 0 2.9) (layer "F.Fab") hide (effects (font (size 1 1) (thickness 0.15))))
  (pad "1" smd rect (at -1.35 -0.95) (size 1.56 0.65) (layers "F.Cu" "F.Paste" "F.Mask") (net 11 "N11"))
  (pad "2" smd rect (at -1.35 0) (size 1.56 0.65) (layers "F.Cu" "F.Paste" "F.Mask") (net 6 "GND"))
  (pad "3" smd rect (at -1.35 0.95) (size 1.56 0.65) (layers "F.Cu" "F.Paste" "F.Mask") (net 10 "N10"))
  (pad "4" smd rect (at 1.35 0.95) (size 1.56 0.65) (layers "F.Cu" "F.Paste" "F.Mask") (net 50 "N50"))
  (pad "5" smd rect (at 1.35 0) (size 1.56 0.65) (layers "F.Cu" "F.Paste" "F.Mask") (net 3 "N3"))
  (pad "6" smd rect (at 1.35 -0.95) (size 1.56 0.65) (layers "F.Cu" "F.Paste" "F.Mask") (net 50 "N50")))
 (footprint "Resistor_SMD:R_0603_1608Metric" (layer "F.Cu") (at 137.16 63.5)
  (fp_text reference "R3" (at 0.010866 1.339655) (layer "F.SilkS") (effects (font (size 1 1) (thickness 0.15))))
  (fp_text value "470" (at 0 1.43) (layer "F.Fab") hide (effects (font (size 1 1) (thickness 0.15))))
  (pad "1" smd roundrect (at -0.825 0) (size 0.8 0.95) (layers "F.Cu" "F.Paste" "F.Mask") (roundrect_rratio 0.25) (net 6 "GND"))
  (pad "2" smd roundrect (at 0.825 0) (size 0.8 0.95) (layers "F.Cu" "F.Paste" "F.Mask") (roundrect_rratio 0.25) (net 9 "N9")))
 (gr_line (start 154.94 142.24) (end 124.46 142.24) (stroke (width 0.1) (type default)) (layer "Edge.Cuts"))
 (gr_line (start 154.94 46.99) (end 154.94 48.26) (stroke (width 0.1) (type default)) (layer "Edge.Cuts"))
 (gr_line (start 124.46 142.24) (end 124.46 46.99) (stroke (width 0.1) (type default)) (layer "Edge.Cuts"))
 (gr_line (start 124.46 46.99) (end 154.94 46.99) (stroke (width 0.1) (type default)) (layer "Edge.Cuts"))
 (gr_line (start 154.94 48.26) (end 154.94 142.24) (stroke (width 0.1) (type default)) (layer "Edge.Cuts"))
 (segment (start 137.16 50.8) (end 139.255 52.895) (width 0.5) (layer "F.Cu") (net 1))
 (segment (start 139.255 52.895) (end 139.255 55.88) (width 0.5) (layer "F.Cu") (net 1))
 (segment (start 131.763604 62.23) (end 131.875 62.118604) (width 0.25) (layer "F.Cu") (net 6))
 (segment (start 139.89724 60.96) (end 138.53 59.59276) (width 0.25) (layer "F.Cu") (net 6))
 (segment (start 140.182265 63.5) (end 140.182265 61.245025) (width 0.25) (layer "F.Cu") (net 6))
 (segment (start 138.14967 60.96) (end 137.81 61.29967) (width 0.25) (layer "F.Cu") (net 6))
 (segment (start 129.461802 60.881802) (end 129.09 61.253604) (width 0.25) (layer "F.Cu") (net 6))
 (segment (start 135.785 49.635) (end 135.995 49.425) (width 0.25) (layer "F.Cu") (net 6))
 (segment (start 140.182265 64.287735) (end 140.182265 63.5) (width 0.25) (layer "F.Cu") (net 6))
 (segment (start 137.81 62.36033) (end 137.81 61.83) (width 0.25) (layer "F.Cu") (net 6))
 (segment (start 137.81 61.29967) (end 137.81 61.83) (width 0.25) (layer "F.Cu") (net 6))
 (segment (start 128.18 59.6) (end 128.18 52.16) (width 0.25) (layer "F.Cu") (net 6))
 (segment (start 135.995 49.425) (end 140.865 49.425) (width 0.25) (layer "F.Cu") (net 6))
 (segment (start 129.461802 60.881802) (end 128.18 59.6) (width 0.25) (layer "F.Cu") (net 6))
 (segment (start 139.25 65.22) (end 140.97 66.94) (width 0.25) (layer "F.Cu") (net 6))
 (segment (start 139.25 65.22) (end 140.182265 64.287735) (width 0.25) (layer "F.Cu") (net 6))
 (segment (start 130.73 62.23) (end 131.763604 62.23) (width 0.25) (layer "F.Cu") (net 6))
 (segment (start 136.335 63.5) (end 136.551396 63.5) (width 0.25) (layer "F.Cu") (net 6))
 (segment (start 129.99 65.22) (end 139.25 65.22) (width 0.25) (layer "F.Cu") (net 6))
 (segment (start 136.551396 63.5) (end 137.351396 62.7) (width 0.25) (layer "F.Cu") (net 6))
 (segment (start 131.875 62.118604) (end 131.875 60.755) (width 0.25) (layer "F.Cu") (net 6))
 (segment (start 138.53 54.71) (end 135.785 51.965) (width 0.25) (layer "F.Cu") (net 6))
 (segment (start 137.47033 62.7) (end 137.81 62.36033) (width 0.25) (layer "F.Cu") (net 6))
 (segment (start 139.89724 60.96) (end 138.14967 60.96) (width 0.25) (layer "F.Cu") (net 6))
 (segment (start 140.865 49.425) (end 142.24 50.8) (width 0.25) (layer "F.Cu") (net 6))
 (segment (start 129.09 64.32) (end 129.99 65.22) (width 0.25) (layer "F.Cu") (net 6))
 (segment (start 128.18 52.16) (end 129.54 50.8) (width 0.25) (layer "F.Cu") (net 6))
 (segment (start 140.97 66.94) (end 140.97 69.85) (width 0.25) (layer "F.Cu") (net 6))
 (segment (start 137.351396 62.7) (end 137.47033 62.7) (width 0.25) (layer "F.Cu") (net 6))
 (segment (start 140.182265 61.245025) (end 139.89724 60.96) (width 0.25) (layer "F.Cu") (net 6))
 (segment (start 131.875 60.755) (end 131.75 60.63) (width 0.25) (layer "F.Cu") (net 6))
 (segment (start 135.785 51.965) (end 135.785 49.635) (width 0.25) (layer "F.Cu") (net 6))
 (segment (start 138.53 59.59276) (end 138.53 54.71) (width 0.25) (layer "F.Cu") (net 6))
 (segment (start 131.75 60.63) (end 129.713604 60.63) (width 0.25) (layer "F.Cu") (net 6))
 (segment (start 129.09 61.253604) (end 129.09 64.32) (width 0.25) (layer "F.Cu") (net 6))
 (segment (start 129.713604 60.63) (end 129.461802 60.881802) (width 0.25) (layer "F.Cu") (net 6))
 (segment (start 139.7 129.54) (end 130.81 138.43) (width 0.5) (layer "F.Cu") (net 7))
 (segment (start 139.7 95.51) (end 139.7 129.54) (width 0.5) (layer "F.Cu") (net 7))
 (segment (start 151.3775 83.8325) (end 139.7 95.51) (width 0.5) (layer "F.Cu") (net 7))
 (segment (start 137.605 55.88) (end 134.725 53) (width 0.25) (layer "F.Cu") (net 8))
 (segment (start 135.89 60.598173) (end 135.476827 60.185) (width 0.17) (layer "F.Cu") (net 8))
 (segment (start 134.725 49.761828) (end 134.388172 49.425) (width 0.25) (layer "F.Cu") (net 8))
 (segment (start 136.76 61.83) (end 135.89 60.96) (width 0.17) (layer "F.Cu") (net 8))
 (segment (start 131.975 49.635) (end 131.975 56.683173) (width 0.25) (layer "F.Cu") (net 8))
 (segment (start 131.975 56.683173) (end 135.476827 60.185) (width 0.25) (layer "F.Cu") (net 8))
 (segment (start 134.725 53) (end 134.725 49.761828) (width 0.25) (layer "F.Cu") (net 8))
 (segment (start 137.168608 56.316392) (end 137.605 55.88) (width 0.25) (layer "F.Cu") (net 8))
 (segment (start 137.16 61.83) (end 136.76 61.83) (width 0.17) (layer "F.Cu") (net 8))
 (segment (start 137.168608 57.943069) (end 137.168608 56.316392) (width 0.25) (layer "F.Cu") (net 8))
 (segment (start 134.388172 49.425) (end 132.185 49.425) (width 0.25) (layer "F.Cu") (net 8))
 (segment (start 135.89 60.96) (end 135.89 60.598173) (width 0.17) (layer "F.Cu") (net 8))
 (segment (start 132.185 49.425) (end 131.975 49.635) (width 0.25) (layer "F.Cu") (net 8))
 (segment (start 137.16 59.501677) (end 137.168608 59.493069) (width 0.2) (layer "F.Cu") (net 4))
 (segment (start 133.35 50.8) (end 133.35 55.4575) (width 0.5) (layer "F.Cu") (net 4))
 (segment (start 133.35 55.4575) (end 135.0425 57.15) (width 0.5) (layer "F.Cu") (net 4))
 (segment (start 135.0425 57.15) (end 135.0425 57.366961) (width 0.5) (layer "F.Cu") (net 4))
 (segment (start 135.0425 57.366961) (end 137.168608 59.493069) (width 0.5) (layer "F.Cu") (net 4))
 (segment (start 137.16 59.501677) (end 137.16 61.28) (width 0.5) (layer "F.Cu") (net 4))
 (segment (start 152.975 50.105) (end 152.975 135.655) (width 0.25) (layer "F.Cu") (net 20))
 (segment (start 152.295 49.425) (end 152.975 50.105) (width 0.25) (layer "F.Cu") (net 20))
 (segment (start 150.2 138.43) (end 148.59 138.43) (width 0.25) (layer "F.Cu") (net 20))
 (segment (start 147.425 49.425) (end 152.295 49.425) (width 0.25) (layer "F.Cu") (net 20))
 (segment (start 152.975 135.655) (end 150.2 138.43) (width 0.25) (layer "F.Cu") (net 20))
 (segment (start 146.05 50.8) (end 147.425 49.425) (width 0.25) (layer "F.Cu") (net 20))
 (segment (start 138.46 63.025) (end 138.46 62.255) (width 0.25) (layer "F.Cu") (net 9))
 (segment (start 137.985 63.5) (end 138.46 63.025) (width 0.25) (layer "F.Cu") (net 9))
 (segment (start 135.89 62.386396) (end 135.89 62.23) (width 0.25) (layer "F.Cu") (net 3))
 (segment (start 135.89 62.23) (end 135.915 62.255) (width 0.25) (layer "F.Cu") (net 3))
 (segment (start 132.325 62.155) (end 132.4 62.23) (width 0.25) (layer "F.Cu") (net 3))
 (segment (start 134.446396 63.83) (end 135.89 62.386396) (width 0.25) (layer "F.Cu") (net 3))
 (segment (start 132.4 62.23) (end 132.08 62.55) (width 0.25) (layer "F.Cu") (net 3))
 (segment (start 129.1175 57.15) (end 132.325 60.3575) (width 0.25) (layer "F.Cu") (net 3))
 (segment (start 132.08 63.585) (end 132.325 63.83) (width 0.25) (layer "F.Cu") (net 3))
 (segment (start 135.915 62.255) (end 137.16 62.255) (width 0.25) (layer "F.Cu") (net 3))
 (segment (start 132.325 63.83) (end 134.446396 63.83) (width 0.25) (layer "F.Cu") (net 3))
 (segment (start 132.325 60.3575) (end 132.325 62.155) (width 0.25) (layer "F.Cu") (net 3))
 (segment (start 132.4 62.23) (end 133.43 62.23) (width 0.25) (layer "F.Cu") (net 3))
 (segment (start 132.08 62.55) (end 132.08 63.585) (width 0.25) (layer "F.Cu") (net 3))
 (segment (start 130.73 61.28) (end 129.7 61.28) (width 0.25) (layer "F.Cu") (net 11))
 (segment (start 130.565 64.77) (end 138.568858 64.77) (width 0.25) (layer "F.Cu") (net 11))
 (segment (start 129.7 61.28) (end 129.54 61.44) (width 0.25) (layer "F.Cu") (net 11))
 (segment (start 129.54 61.44) (end 129.54 63.745) (width 0.25) (layer "F.Cu") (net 11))
 (segment (start 138.568858 64.77) (end 139.732265 63.606593) (width 0.25) (layer "F.Cu") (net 11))
 (segment (start 138.46929 61.42071) (end 138.46 61.43) (width 0.17) (layer "F.Cu") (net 11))
 (segment (start 139.732265 61.431421) (end 139.721554 61.42071) (width 0.17) (layer "F.Cu") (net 11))
 (segment (start 139.732265 63.606593) (end 139.732265 61.431421) (width 0.25) (layer "F.Cu") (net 11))
 (segment (start 129.54 63.745) (end 130.565 64.77) (width 0.25) (layer "F.Cu") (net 11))
 (segment (start 139.721554 61.42071) (end 138.46929 61.42071) (width 0.17) (layer "F.Cu") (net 11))
 (segment (start 138.46071 61.83071) (end 138.46 61.83) (width 0.17) (layer "F.Cu") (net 10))
 (segment (start 139.272944 63.429518) (end 139.272944 61.83071) (width 0.25) (layer "F.Cu") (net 10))
 (segment (start 130.73 63.18) (end 131.85 64.3) (width 0.25) (layer "F.Cu") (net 10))
 (segment (start 138.402462 64.3) (end 139.272944 63.429518) (width 0.25) (layer "F.Cu") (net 10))
 (segment (start 139.272944 61.83071) (end 138.46071 61.83071) (width 0.17) (layer "F.Cu") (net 10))
 (segment (start 131.85 64.3) (end 138.402462 64.3) (width 0.25) (layer "F.Cu") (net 10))
 (segment (start 134.62 63.02) (end 134.46 63.18) (width 0.25) (layer "F.Cu") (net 50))
 (segment (start 133.43 61.28) (end 134.46 61.28) (width 0.25) (layer "F.Cu") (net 50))
 (segment (start 134.46 61.28) (end 134.62 61.44) (width 0.25) (layer "F.Cu") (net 50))
 (segment (start 134.46 63.18) (end 133.43 63.18) (width 0.25) (layer "F.Cu") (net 50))
 (segment (start 134.62 61.44) (end 134.62 63.02) (width 0.25) (layer "F.Cu") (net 50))
 (segment (start 135.89 69.85) (end 130.81 74.93) (width 0.25) (layer "F.Cu") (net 18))
 (segment (start 130.81 74.93) (end 130.81 90.17) (width 0.25) (layer "F.Cu") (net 18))
 (segment (start 138.43 69.85) (end 132.347251 75.932749) (width 0.25) (layer "F.Cu") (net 17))
 (segment (start 132.347251 75.932749) (end 132.347251 91.172749) (width 0.25) (layer "F.Cu") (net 17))
 (segment (start 132.347251 91.172749) (end 130.81 92.71) (width 0.25) (layer "F.Cu") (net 17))
 (segment (start 146.05 69.85) (end 146.05 82.44) (width 0.25) (layer "F.Cu") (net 15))
 (segment (start 146.05 82.44) (end 142.767327 85.722673) (width 0.25) (layer "F.Cu") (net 15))
 (segment (start 139.270463 85.722673) (end 138.335 86.658136) (width 0.25) (layer "F.Cu") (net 15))
 (segment (start 142.767327 85.722673) (end 139.270463 85.722673) (width 0.25) (layer "F.Cu") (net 15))
 (segment (start 138.335 86.658136) (end 138.335 120.745) (width 0.25) (layer "F.Cu") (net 15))
 (segment (start 138.335 120.745) (end 130.81 128.27) (width 0.25) (layer "F.Cu") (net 15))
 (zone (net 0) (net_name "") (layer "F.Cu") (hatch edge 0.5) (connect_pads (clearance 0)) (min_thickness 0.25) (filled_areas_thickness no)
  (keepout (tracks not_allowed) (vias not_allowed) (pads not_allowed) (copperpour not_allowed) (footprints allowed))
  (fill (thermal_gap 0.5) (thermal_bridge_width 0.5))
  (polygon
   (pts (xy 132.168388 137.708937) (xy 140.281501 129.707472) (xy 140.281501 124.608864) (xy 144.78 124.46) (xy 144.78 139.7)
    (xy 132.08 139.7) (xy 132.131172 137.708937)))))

